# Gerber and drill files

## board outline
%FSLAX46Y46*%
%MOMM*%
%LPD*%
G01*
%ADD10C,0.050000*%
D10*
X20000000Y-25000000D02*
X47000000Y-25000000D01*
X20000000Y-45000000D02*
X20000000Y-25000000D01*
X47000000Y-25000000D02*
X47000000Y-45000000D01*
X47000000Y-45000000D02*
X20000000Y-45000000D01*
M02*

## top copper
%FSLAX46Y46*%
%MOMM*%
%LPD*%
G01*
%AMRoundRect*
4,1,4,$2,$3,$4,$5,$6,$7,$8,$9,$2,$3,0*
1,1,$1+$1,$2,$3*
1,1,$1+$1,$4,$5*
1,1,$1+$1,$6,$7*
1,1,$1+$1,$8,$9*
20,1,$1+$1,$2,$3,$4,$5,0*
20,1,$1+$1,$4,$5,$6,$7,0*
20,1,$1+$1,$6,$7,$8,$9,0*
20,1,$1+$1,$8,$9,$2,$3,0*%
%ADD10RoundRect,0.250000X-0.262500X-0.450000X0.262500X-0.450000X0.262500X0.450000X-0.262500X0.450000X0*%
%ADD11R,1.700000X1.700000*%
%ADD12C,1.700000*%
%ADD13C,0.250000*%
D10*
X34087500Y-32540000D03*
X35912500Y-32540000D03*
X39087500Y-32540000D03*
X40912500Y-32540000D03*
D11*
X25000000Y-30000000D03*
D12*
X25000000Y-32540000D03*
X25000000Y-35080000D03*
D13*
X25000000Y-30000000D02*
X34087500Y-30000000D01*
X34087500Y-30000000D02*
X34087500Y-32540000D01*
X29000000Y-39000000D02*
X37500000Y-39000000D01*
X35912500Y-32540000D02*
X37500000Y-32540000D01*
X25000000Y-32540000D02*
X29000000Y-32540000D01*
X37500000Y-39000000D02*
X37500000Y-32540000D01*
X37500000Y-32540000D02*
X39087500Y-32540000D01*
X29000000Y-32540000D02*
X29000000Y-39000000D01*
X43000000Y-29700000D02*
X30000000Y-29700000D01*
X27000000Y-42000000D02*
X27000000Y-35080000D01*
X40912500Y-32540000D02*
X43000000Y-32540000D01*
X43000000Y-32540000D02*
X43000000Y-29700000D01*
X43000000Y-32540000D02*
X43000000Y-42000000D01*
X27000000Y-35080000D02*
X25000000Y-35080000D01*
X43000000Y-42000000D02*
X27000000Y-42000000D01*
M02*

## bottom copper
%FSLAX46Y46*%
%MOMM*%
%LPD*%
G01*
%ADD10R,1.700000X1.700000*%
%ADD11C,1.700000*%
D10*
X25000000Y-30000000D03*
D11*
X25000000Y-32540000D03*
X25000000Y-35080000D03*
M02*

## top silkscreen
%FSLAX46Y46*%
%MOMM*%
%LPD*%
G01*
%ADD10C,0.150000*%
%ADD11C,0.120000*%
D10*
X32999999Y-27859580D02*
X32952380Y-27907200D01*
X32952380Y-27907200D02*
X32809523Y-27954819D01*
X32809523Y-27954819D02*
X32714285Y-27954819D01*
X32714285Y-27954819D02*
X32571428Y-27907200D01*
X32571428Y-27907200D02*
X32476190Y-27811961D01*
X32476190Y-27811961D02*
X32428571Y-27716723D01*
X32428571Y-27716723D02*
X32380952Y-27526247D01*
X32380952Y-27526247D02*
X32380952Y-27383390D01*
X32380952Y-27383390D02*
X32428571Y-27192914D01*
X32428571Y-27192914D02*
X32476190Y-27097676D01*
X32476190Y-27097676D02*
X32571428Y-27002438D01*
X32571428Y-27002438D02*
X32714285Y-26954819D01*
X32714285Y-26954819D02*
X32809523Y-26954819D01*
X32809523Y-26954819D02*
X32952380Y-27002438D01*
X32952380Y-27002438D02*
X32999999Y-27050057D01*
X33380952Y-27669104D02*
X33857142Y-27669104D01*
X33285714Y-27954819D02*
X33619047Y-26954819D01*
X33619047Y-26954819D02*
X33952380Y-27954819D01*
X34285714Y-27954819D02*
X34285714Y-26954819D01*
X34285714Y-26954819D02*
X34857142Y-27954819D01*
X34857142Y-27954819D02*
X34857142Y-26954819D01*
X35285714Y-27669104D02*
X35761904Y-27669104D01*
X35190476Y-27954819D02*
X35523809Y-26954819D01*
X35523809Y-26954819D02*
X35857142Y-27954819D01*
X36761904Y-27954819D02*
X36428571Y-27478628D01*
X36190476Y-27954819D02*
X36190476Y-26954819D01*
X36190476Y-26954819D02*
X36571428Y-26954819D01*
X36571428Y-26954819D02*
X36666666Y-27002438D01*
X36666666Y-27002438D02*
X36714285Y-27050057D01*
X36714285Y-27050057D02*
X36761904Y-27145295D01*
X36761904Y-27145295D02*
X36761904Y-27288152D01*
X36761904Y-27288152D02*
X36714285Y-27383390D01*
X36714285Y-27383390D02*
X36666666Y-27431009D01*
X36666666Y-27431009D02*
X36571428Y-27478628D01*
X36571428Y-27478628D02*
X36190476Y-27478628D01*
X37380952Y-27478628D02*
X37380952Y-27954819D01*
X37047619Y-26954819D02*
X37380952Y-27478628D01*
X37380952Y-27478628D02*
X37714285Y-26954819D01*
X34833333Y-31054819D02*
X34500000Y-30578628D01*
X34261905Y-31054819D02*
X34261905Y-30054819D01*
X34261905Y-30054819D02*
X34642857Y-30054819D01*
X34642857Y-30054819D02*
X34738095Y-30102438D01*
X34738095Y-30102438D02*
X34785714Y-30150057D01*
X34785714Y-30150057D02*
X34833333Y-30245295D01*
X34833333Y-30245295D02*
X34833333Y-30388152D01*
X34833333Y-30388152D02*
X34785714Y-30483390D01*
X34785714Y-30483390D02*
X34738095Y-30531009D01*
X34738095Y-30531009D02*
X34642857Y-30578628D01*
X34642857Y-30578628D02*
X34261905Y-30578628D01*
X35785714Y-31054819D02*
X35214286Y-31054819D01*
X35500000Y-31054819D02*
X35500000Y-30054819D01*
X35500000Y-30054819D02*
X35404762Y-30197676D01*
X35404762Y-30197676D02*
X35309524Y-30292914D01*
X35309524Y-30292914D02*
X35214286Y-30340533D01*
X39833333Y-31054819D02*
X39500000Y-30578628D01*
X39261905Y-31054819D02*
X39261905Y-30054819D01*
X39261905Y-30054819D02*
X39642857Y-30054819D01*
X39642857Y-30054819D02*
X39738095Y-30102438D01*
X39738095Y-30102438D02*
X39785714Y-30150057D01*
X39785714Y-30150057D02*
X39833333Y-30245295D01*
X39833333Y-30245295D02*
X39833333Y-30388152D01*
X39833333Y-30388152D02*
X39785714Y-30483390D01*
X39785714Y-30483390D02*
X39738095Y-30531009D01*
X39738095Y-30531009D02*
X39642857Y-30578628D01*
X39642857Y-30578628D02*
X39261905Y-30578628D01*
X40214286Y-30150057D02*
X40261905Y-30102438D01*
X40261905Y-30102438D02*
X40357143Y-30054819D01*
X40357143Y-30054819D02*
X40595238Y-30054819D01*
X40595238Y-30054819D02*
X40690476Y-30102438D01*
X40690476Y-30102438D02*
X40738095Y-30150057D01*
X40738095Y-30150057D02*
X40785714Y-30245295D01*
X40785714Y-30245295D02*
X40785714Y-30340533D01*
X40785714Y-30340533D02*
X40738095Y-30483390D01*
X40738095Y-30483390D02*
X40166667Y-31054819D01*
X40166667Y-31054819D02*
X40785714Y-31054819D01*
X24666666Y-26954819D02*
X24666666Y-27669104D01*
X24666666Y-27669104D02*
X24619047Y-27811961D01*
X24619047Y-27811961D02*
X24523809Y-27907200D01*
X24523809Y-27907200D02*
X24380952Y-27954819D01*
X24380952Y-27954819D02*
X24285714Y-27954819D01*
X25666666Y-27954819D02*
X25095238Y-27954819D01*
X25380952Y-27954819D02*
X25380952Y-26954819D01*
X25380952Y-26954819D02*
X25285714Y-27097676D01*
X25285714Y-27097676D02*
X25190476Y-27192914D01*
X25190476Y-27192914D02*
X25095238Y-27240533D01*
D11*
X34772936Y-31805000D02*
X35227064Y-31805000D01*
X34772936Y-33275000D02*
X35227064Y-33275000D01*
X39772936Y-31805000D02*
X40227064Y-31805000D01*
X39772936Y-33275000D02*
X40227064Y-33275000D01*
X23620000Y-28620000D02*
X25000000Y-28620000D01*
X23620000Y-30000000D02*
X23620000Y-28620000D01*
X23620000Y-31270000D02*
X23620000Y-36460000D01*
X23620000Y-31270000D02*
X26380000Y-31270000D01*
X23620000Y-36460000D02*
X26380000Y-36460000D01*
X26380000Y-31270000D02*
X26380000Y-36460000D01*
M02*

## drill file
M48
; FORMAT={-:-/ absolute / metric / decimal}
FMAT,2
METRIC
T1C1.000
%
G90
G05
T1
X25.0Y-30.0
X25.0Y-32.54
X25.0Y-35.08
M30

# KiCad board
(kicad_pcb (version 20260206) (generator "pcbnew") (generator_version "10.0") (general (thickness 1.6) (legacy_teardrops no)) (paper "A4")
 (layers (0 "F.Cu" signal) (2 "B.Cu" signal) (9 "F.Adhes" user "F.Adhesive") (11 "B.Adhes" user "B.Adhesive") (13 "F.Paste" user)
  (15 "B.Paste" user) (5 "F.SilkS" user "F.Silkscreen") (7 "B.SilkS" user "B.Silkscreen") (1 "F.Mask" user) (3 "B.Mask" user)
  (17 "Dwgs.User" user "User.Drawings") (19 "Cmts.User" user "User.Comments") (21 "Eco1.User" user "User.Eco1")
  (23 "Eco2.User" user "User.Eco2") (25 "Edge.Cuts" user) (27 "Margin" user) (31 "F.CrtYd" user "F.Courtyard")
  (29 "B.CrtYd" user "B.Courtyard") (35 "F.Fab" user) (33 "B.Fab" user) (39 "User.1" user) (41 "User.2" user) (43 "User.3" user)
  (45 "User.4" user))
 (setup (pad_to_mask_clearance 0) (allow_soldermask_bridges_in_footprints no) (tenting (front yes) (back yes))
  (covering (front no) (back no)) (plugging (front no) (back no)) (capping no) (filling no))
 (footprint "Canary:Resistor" (layer "F.Cu") (at 35 32.54)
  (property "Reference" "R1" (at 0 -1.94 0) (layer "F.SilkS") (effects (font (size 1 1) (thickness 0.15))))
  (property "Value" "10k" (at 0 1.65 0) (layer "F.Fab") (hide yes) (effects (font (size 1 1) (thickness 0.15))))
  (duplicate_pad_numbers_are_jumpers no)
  (fp_line (start -0.227064 -0.735) (end 0.227064 -0.735) (stroke (width 0.12) (type solid)) (layer "F.SilkS"))
  (fp_line (start -0.227064 0.735) (end 0.227064 0.735) (stroke (width 0.12) (type solid)) (layer "F.SilkS"))
  (pad "1" smd roundrect (at -0.9125 0) (size 1.025 1.4) (layers "F.Cu" "F.Mask" "F.Paste") (roundrect_rratio 0.243902) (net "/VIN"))
  (pad "2" smd roundrect (at 0.9125 0) (size 1.025 1.4) (layers "F.Cu" "F.Mask" "F.Paste") (roundrect_rratio 0.243902) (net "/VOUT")))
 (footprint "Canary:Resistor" (layer "F.Cu") (at 40 32.54)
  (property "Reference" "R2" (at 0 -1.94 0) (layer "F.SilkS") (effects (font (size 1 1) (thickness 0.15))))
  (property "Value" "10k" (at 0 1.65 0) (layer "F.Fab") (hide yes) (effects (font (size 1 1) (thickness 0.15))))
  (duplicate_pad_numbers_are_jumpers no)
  (fp_line (start -0.227064 -0.735) (end 0.227064 -0.735) (stroke (width 0.12) (type solid)) (layer "F.SilkS"))
  (fp_line (start -0.227064 0.735) (end 0.227064 0.735) (stroke (width 0.12) (type solid)) (layer "F.SilkS"))
  (pad "1" smd roundrect (at -0.9125 0) (size 1.025 1.4) (layers "F.Cu" "F.Mask" "F.Paste") (roundrect_rratio 0.243902) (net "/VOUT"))
  (pad "2" smd roundrect (at 0.9125 0) (size 1.025 1.4) (layers "F.Cu" "F.Mask" "F.Paste") (roundrect_rratio 0.243902) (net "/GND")))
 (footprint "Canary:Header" (layer "F.Cu") (at 25 30)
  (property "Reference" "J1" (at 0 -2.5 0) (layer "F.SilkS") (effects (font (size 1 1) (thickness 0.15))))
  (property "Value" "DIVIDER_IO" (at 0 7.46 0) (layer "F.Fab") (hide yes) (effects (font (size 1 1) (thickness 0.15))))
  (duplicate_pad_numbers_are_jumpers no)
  (fp_line (start -1.38 -1.38) (end 0 -1.38) (stroke (width 0.12) (type solid)) (layer "F.SilkS"))
  (fp_line (start -1.38 0) (end -1.38 -1.38) (stroke (width 0.12) (type solid)) (layer "F.SilkS"))
  (fp_line (start -1.38 1.27) (end -1.38 6.46) (stroke (width 0.12) (type solid)) (layer "F.SilkS"))
  (fp_line (start -1.38 1.27) (end 1.38 1.27) (stroke (width 0.12) (type solid)) (layer "F.SilkS"))
  (fp_line (start -1.38 6.46) (end 1.38 6.46) (stroke (width 0.12) (type solid)) (layer "F.SilkS"))
  (fp_line (start 1.38 1.27) (end 1.38 6.46) (stroke (width 0.12) (type solid)) (layer "F.SilkS"))
  (pad "1" thru_hole rect (at 0 0) (size 1.7 1.7) (drill 1) (layers "*.Cu" "*.Mask") (remove_unused_layers no) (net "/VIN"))
  (pad "2" thru_hole circle (at 0 2.54) (size 1.7 1.7) (drill 1) (layers "*.Cu" "*.Mask") (remove_unused_layers no) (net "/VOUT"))
  (pad "3" thru_hole circle (at 0 5.08) (size 1.7 1.7) (drill 1) (layers "*.Cu" "*.Mask") (remove_unused_layers no) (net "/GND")))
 (gr_line (start 20 25) (end 47 25) (stroke (width 0.05) (type default)) (layer "Edge.Cuts"))
 (gr_line (start 20 45) (end 20 25) (stroke (width 0.05) (type default)) (layer "Edge.Cuts"))
 (gr_line (start 47 25) (end 47 45) (stroke (width 0.05) (type default)) (layer "Edge.Cuts"))
 (gr_line (start 47 45) (end 20 45) (stroke (width 0.05) (type default)) (layer "Edge.Cuts"))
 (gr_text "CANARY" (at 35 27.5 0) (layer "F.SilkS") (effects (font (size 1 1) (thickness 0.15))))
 (segment (start 25 30) (end 34.0875 30) (width 0.25) (layer "F.Cu") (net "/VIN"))
 (segment (start 34.0875 30) (end 34.0875 32.54) (width 0.25) (layer "F.Cu") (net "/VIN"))
 (segment (start 29 39) (end 37.5 39) (width 0.25) (layer "F.Cu") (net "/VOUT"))
 (segment (start 35.9125 32.54) (end 37.5 32.54) (width 0.25) (layer "F.Cu") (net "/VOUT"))
 (segment (start 25 32.54) (end 29 32.54) (width 0.25) (layer "F.Cu") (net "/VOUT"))
 (segment (start 37.5 39) (end 37.5 32.54) (width 0.25) (layer "F.Cu") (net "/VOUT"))
 (segment (start 37.5 32.54) (end 39.0875 32.54) (width 0.25) (layer "F.Cu") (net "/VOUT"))
 (segment (start 29 32.54) (end 29 39) (width 0.25) (layer "F.Cu") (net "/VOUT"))
 (segment (start 43 29.7) (end 30 29.7) (width 0.25) (layer "F.Cu") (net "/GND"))
 (segment (start 27 42) (end 27 35.08) (width 0.25) (layer "F.Cu") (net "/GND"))
 (segment (start 40.9125 32.54) (end 43 32.54) (width 0.25) (layer "F.Cu") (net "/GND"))
 (segment (start 43 32.54) (end 43 29.7) (width 0.25) (layer "F.Cu") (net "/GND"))
 (segment (start 43 32.54) (end 43 42) (width 0.25) (layer "F.Cu") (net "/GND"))
 (segment (start 27 35.08) (end 25 35.08) (width 0.25) (layer "F.Cu") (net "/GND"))
 (segment (start 43 42) (end 27 42) (width 0.25) (layer "F.Cu") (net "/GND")))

